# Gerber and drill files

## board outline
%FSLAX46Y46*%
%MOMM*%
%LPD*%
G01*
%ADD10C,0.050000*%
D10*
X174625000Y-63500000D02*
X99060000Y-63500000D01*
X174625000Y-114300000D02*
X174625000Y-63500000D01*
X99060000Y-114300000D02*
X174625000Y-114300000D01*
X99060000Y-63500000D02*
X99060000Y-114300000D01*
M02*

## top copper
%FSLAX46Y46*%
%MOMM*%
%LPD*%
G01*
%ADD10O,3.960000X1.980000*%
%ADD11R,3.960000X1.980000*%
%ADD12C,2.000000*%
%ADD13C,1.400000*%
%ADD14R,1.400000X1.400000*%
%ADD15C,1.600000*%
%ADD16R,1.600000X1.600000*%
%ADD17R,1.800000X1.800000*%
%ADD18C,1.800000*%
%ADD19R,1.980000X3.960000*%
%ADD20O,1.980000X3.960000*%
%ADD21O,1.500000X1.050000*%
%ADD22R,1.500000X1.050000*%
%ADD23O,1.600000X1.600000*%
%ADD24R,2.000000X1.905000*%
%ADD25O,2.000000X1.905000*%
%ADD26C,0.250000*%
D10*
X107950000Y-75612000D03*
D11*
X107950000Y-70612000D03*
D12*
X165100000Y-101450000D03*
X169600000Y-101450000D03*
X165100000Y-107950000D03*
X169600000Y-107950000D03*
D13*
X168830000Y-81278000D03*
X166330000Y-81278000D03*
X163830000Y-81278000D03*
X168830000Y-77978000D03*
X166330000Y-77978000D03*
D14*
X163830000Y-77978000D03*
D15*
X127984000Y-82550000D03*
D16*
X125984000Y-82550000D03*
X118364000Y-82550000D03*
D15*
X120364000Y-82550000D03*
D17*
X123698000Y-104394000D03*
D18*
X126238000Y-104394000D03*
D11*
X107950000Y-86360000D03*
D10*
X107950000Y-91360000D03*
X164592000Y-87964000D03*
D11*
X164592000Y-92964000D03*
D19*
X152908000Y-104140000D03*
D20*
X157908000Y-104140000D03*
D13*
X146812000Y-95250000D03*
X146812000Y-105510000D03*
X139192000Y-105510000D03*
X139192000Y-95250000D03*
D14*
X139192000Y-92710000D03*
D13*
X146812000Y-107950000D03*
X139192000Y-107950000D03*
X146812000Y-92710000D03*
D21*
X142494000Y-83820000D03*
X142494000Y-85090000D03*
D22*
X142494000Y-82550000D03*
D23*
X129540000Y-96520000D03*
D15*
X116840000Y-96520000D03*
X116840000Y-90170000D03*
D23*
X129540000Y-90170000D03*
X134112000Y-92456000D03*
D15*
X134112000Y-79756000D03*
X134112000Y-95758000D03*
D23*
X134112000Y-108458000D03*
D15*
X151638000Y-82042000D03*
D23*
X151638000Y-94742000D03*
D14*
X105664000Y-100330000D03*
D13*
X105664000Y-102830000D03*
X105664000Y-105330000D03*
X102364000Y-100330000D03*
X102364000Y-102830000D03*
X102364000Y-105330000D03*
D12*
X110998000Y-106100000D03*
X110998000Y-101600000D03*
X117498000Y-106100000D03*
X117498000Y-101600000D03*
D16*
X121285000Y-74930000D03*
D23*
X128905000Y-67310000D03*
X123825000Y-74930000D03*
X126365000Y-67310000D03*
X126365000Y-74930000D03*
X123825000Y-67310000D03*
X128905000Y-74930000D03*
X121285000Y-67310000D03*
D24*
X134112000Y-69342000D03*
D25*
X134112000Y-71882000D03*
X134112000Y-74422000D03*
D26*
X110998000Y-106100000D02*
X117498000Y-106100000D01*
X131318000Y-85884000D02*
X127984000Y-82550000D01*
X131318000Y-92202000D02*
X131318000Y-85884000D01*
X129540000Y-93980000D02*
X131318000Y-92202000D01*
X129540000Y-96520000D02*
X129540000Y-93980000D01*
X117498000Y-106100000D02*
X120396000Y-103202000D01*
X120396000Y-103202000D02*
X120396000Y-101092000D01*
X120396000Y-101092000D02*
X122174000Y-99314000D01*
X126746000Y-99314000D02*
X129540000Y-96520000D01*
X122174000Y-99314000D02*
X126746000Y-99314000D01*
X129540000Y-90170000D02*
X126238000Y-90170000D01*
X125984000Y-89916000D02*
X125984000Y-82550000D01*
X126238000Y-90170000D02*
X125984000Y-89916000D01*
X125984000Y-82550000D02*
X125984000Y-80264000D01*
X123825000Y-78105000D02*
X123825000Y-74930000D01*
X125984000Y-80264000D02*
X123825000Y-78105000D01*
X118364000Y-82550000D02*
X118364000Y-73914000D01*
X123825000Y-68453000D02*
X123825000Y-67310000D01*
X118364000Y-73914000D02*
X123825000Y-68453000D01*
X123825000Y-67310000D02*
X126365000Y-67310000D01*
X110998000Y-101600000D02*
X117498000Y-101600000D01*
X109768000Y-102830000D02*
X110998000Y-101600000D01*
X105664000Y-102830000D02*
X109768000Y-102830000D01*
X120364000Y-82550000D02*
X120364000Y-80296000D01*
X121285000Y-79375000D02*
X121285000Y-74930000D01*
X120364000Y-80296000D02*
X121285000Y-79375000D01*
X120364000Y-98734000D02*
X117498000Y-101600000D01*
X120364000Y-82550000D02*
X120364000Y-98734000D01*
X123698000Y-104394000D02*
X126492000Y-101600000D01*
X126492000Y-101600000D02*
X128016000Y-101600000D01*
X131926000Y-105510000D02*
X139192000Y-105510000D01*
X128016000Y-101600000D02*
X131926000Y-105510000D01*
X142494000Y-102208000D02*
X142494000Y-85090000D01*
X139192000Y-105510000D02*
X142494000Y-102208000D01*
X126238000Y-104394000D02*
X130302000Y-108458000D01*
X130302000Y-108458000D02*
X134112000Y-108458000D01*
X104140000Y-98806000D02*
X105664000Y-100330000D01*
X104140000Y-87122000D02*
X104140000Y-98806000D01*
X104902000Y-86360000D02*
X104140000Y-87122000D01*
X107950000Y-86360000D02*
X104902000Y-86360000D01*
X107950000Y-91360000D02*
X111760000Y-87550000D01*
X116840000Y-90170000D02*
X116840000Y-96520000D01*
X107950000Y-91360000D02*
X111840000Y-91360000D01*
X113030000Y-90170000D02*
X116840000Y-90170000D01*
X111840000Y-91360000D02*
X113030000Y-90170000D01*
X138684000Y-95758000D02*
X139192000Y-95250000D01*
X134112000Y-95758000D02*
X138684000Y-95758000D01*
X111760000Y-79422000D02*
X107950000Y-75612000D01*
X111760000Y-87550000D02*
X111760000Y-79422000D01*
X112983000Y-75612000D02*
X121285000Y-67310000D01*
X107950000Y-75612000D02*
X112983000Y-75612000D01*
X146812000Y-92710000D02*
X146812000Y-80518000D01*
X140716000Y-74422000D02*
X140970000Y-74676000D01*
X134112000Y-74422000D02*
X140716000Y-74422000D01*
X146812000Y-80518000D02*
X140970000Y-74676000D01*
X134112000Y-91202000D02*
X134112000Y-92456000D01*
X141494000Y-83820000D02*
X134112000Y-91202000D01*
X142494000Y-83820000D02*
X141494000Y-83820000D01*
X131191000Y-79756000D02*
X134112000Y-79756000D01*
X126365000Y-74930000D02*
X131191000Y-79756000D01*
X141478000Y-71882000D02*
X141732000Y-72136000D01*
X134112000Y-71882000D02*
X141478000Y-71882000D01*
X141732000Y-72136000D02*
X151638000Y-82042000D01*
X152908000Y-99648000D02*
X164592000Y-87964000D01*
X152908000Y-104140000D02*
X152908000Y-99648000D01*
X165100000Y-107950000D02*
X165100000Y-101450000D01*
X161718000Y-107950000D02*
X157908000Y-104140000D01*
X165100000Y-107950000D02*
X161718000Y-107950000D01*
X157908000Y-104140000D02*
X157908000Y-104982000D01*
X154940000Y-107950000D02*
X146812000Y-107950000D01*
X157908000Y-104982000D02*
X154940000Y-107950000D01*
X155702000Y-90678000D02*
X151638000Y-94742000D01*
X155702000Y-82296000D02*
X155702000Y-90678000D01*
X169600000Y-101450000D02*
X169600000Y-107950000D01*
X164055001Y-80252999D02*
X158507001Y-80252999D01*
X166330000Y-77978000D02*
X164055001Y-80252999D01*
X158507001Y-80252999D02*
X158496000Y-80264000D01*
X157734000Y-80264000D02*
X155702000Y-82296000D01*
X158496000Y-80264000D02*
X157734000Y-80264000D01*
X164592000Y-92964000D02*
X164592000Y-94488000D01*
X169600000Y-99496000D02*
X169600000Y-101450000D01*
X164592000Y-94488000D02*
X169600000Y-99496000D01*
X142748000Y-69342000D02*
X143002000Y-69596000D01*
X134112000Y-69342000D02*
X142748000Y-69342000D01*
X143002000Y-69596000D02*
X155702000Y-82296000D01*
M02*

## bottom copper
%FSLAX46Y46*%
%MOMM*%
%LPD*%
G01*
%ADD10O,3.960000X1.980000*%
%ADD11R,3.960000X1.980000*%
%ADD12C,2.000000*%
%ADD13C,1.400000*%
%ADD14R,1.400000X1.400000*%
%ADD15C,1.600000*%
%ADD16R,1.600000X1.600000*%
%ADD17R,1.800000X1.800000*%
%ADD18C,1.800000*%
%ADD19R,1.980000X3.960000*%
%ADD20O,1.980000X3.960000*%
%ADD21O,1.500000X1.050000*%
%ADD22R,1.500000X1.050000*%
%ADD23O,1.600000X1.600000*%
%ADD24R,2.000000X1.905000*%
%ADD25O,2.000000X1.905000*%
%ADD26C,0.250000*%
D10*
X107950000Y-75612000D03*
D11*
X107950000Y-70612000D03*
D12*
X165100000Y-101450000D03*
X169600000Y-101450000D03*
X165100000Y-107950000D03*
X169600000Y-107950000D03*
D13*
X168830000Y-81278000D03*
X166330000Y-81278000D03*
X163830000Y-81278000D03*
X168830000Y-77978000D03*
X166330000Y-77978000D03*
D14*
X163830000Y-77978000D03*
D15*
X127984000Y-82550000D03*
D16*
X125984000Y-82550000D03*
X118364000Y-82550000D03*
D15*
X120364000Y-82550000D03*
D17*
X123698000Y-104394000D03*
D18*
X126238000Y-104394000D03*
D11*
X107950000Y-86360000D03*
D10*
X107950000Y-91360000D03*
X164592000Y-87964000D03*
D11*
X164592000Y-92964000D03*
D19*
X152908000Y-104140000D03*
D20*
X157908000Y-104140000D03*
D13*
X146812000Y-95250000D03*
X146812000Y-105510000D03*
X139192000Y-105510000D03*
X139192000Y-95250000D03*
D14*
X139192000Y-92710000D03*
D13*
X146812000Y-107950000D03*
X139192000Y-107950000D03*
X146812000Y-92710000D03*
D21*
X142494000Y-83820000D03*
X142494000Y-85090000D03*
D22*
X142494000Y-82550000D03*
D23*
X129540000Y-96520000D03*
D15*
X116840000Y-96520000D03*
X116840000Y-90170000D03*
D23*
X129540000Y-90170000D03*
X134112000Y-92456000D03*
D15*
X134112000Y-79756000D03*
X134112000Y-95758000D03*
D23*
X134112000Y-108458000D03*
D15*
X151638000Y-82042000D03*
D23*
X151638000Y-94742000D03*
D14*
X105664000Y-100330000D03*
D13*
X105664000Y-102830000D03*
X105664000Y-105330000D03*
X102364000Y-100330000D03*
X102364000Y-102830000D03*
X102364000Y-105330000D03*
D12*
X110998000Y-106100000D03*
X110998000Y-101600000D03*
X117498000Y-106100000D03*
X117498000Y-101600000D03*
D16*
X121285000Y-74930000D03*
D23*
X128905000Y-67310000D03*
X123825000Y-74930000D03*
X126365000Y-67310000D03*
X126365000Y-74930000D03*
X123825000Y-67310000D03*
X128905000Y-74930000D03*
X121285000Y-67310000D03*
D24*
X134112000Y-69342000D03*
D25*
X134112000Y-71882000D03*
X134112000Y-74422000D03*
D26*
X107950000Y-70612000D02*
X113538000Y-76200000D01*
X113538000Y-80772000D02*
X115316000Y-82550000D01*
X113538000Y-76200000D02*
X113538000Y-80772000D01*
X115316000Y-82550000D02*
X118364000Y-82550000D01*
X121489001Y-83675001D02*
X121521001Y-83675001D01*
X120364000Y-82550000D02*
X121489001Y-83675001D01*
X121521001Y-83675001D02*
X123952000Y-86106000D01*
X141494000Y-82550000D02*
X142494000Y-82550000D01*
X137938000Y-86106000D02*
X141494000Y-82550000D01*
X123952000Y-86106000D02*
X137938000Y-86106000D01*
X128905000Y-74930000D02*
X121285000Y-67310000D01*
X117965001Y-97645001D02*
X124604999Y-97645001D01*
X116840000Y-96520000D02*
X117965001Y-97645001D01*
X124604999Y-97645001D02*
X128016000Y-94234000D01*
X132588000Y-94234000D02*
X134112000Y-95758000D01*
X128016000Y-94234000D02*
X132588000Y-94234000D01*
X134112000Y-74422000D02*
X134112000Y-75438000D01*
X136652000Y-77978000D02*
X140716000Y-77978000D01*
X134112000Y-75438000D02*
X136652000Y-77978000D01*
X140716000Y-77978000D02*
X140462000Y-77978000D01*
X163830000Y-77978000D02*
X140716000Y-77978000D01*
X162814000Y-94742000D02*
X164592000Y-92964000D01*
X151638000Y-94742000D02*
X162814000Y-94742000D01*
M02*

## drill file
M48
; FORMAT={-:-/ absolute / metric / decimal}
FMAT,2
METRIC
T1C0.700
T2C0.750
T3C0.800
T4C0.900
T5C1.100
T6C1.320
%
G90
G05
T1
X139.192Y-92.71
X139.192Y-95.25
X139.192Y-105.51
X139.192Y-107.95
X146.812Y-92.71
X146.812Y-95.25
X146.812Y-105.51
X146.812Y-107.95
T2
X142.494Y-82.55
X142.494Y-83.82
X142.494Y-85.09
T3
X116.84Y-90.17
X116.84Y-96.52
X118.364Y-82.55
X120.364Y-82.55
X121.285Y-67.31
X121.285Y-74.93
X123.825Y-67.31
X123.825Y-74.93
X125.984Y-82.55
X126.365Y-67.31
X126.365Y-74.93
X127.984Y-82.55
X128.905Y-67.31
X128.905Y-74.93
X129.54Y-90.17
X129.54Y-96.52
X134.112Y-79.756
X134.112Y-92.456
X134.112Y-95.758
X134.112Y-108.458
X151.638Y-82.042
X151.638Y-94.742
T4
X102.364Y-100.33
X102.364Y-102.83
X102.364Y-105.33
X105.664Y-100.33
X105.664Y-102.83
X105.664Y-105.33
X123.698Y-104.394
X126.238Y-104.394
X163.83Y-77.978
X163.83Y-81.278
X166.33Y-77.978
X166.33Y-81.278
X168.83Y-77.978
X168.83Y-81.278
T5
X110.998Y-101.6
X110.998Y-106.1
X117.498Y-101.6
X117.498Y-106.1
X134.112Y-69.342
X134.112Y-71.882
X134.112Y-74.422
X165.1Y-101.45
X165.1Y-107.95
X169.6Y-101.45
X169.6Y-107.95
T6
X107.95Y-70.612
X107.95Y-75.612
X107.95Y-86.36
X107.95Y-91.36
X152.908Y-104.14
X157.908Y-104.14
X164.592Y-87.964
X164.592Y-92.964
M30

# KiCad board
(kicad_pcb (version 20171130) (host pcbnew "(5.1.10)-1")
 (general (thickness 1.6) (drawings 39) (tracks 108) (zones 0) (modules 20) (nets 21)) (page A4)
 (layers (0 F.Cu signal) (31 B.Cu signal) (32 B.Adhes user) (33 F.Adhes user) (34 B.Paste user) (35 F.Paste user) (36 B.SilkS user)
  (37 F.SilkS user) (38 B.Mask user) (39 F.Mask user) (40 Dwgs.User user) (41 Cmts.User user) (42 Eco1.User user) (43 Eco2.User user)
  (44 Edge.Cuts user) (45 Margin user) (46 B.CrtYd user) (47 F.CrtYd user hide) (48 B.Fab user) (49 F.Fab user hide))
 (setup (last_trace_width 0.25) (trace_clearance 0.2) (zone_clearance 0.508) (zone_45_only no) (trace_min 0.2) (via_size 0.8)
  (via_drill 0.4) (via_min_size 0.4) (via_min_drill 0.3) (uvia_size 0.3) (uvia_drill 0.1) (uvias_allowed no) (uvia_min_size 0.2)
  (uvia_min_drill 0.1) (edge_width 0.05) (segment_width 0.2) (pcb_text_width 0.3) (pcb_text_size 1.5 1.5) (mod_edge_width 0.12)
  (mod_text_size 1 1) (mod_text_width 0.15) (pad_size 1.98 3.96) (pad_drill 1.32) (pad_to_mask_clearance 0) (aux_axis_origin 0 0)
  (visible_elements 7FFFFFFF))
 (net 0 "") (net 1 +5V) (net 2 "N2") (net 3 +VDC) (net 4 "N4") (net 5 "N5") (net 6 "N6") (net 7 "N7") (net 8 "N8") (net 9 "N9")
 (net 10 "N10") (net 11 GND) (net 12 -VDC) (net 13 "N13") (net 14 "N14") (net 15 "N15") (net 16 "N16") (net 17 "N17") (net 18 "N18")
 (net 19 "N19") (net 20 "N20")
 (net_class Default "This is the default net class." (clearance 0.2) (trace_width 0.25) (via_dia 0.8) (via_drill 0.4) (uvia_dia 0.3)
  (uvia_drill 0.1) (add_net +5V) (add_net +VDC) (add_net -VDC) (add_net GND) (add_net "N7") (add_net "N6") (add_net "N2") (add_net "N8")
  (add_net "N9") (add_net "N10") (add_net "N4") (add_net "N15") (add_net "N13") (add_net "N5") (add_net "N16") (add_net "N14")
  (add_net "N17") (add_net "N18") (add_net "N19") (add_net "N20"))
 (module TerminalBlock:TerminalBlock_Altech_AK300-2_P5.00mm (layer F.Cu) (at 107.95 70.612 270)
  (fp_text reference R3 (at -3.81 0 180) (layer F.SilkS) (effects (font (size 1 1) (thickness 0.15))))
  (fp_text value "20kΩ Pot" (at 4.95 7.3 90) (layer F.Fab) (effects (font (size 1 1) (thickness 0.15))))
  (pad 2 thru_hole oval (at 5 0 270) (size 1.98 3.96) (drill 1.32) (layers *.Cu *.Mask) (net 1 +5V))
  (pad 1 thru_hole rect (at 0 0 270) (size 1.98 3.96) (drill 1.32) (layers *.Cu *.Mask) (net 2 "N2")))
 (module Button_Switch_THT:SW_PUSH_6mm (layer F.Cu) (at 165.1 107.95 90)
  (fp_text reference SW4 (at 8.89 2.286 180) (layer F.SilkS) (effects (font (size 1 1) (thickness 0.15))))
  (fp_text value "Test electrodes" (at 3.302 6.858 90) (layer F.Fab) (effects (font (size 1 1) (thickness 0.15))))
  (pad 1 thru_hole circle (at 6.5 0 180) (size 2 2) (drill 1.1) (layers *.Cu *.Mask) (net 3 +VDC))
  (pad 2 thru_hole circle (at 6.5 4.5 180) (size 2 2) (drill 1.1) (layers *.Cu *.Mask) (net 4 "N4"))
  (pad 1 thru_hole circle (at 0 0 180) (size 2 2) (drill 1.1) (layers *.Cu *.Mask) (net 3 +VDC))
  (pad 2 thru_hole circle (at 0 4.5 180) (size 2 2) (drill 1.1) (layers *.Cu *.Mask) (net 4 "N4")))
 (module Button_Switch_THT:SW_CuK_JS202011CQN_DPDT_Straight (layer F.Cu) (at 163.83 77.978)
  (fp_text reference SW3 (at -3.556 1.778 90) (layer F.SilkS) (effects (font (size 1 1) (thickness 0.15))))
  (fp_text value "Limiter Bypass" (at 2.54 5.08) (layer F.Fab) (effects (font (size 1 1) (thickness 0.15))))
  (pad 6 thru_hole circle (at 5 3.3) (size 1.4 1.4) (drill 0.9) (layers *.Cu *.Mask))
  (pad 5 thru_hole circle (at 2.5 3.3) (size 1.4 1.4) (drill 0.9) (layers *.Cu *.Mask))
  (pad 4 thru_hole circle (at 0 3.3) (size 1.4 1.4) (drill 0.9) (layers *.Cu *.Mask))
  (pad 3 thru_hole circle (at 5 0) (size 1.4 1.4) (drill 0.9) (layers *.Cu *.Mask))
  (pad 2 thru_hole circle (at 2.5 0) (size 1.4 1.4) (drill 0.9) (layers *.Cu *.Mask) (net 4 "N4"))
  (pad 1 thru_hole rect (at 0 0) (size 1.4 1.4) (drill 0.9) (layers *.Cu *.Mask) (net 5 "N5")))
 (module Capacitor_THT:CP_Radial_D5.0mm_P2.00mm (layer F.Cu) (at 125.984 82.55)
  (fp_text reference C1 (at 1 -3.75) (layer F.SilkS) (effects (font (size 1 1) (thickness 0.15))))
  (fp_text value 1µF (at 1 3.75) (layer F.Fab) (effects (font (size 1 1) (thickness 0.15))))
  (pad 2 thru_hole circle (at 2 0) (size 1.6 1.6) (drill 0.8) (layers *.Cu *.Mask) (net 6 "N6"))
  (pad 1 thru_hole rect (at 0 0) (size 1.6 1.6) (drill 0.8) (layers *.Cu *.Mask) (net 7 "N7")))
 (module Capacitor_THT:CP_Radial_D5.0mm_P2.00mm (layer F.Cu) (at 118.364 82.55)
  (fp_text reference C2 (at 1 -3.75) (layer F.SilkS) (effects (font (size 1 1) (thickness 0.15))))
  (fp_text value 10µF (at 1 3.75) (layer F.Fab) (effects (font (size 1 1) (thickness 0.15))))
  (pad 1 thru_hole rect (at 0 0) (size 1.6 1.6) (drill 0.8) (layers *.Cu *.Mask) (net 2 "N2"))
  (pad 2 thru_hole circle (at 2 0) (size 1.6 1.6) (drill 0.8) (layers *.Cu *.Mask) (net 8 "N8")))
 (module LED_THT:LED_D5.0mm (layer F.Cu) (at 123.698 104.394)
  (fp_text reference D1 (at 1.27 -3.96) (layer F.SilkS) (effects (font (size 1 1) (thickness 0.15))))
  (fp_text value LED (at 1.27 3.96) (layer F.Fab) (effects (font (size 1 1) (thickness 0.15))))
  (pad 1 thru_hole rect (at 0 0) (size 1.8 1.8) (drill 0.9) (layers *.Cu *.Mask) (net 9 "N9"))
  (pad 2 thru_hole circle (at 2.54 0) (size 1.8 1.8) (drill 0.9) (layers *.Cu *.Mask) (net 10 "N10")))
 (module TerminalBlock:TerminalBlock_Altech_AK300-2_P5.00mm (layer F.Cu) (at 107.95 86.36 270)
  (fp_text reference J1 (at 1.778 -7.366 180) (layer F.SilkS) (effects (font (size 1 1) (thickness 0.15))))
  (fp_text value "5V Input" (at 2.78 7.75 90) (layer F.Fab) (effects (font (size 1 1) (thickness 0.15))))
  (pad 1 thru_hole rect (at 0 0 270) (size 1.98 3.96) (drill 1.32) (layers *.Cu *.Mask) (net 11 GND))
  (pad 2 thru_hole oval (at 5 0 270) (size 1.98 3.96) (drill 1.32) (layers *.Cu *.Mask) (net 1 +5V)))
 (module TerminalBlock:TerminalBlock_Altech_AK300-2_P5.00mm (layer F.Cu) (at 164.592 92.964 90)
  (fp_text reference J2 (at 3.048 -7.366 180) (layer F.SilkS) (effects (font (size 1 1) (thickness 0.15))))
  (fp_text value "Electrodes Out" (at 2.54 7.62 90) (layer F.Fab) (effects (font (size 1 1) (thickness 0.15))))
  (pad 2 thru_hole oval (at 5 0 90) (size 1.98 3.96) (drill 1.32) (layers *.Cu *.Mask) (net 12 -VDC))
  (pad 1 thru_hole rect (at 0 0 90) (size 1.98 3.96) (drill 1.32) (layers *.Cu *.Mask) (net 4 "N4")))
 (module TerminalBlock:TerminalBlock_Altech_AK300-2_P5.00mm (layer F.Cu) (at 152.908 104.14)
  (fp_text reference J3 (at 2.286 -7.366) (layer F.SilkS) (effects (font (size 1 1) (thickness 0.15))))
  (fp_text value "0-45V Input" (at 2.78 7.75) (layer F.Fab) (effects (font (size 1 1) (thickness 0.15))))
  (pad 1 thru_hole rect (at 0 0) (size 1.98 3.96) (drill 1.32) (layers *.Cu *.Mask) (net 12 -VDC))
  (pad 2 thru_hole oval (at 5 0) (size 1.98 3.96) (drill 1.32) (layers *.Cu *.Mask) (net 3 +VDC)))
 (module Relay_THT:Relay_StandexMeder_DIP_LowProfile (layer F.Cu) (at 139.192 92.71)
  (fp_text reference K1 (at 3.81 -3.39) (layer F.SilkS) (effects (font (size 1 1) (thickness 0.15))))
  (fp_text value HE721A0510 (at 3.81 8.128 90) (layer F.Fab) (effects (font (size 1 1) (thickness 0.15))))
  (pad 13 thru_hole circle (at 7.62 2.54) (size 1.4 1.4) (drill 0.7) (layers *.Cu *.Mask) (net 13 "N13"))
  (pad 9 thru_hole circle (at 7.62 12.8) (size 1.4 1.4) (drill 0.7) (layers *.Cu *.Mask) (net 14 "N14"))
  (pad 6 thru_hole circle (at 0 12.8) (size 1.4 1.4) (drill 0.7) (layers *.Cu *.Mask) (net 9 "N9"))
  (pad 2 thru_hole circle (at 0 2.54) (size 1.4 1.4) (drill 0.7) (layers *.Cu *.Mask) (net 1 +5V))
  (pad 1 thru_hole rect (at 0 0) (size 1.4 1.4) (drill 0.7) (layers *.Cu *.Mask) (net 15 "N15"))
  (pad 8 thru_hole circle (at 7.62 15.24) (size 1.4 1.4) (drill 0.7) (layers *.Cu *.Mask) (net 3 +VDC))
  (pad 7 thru_hole circle (at 0 15.24) (size 1.4 1.4) (drill 0.7) (layers *.Cu *.Mask) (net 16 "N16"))
  (pad 14 thru_hole circle (at 7.62 0) (size 1.4 1.4) (drill 0.7) (layers *.Cu *.Mask) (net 5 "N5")))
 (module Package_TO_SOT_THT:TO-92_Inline (layer F.Cu) (at 142.494 82.55 270)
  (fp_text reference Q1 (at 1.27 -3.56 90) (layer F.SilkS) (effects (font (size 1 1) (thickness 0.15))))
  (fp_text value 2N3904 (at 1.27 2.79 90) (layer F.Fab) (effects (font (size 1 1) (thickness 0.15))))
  (pad 2 thru_hole oval (at 1.27 0 270) (size 1.05 1.5) (drill 0.75) (layers *.Cu *.Mask) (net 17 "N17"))
  (pad 3 thru_hole oval (at 2.54 0 270) (size 1.05 1.5) (drill 0.75) (layers *.Cu *.Mask) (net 9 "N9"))
  (pad 1 thru_hole rect (at 0 0 270) (size 1.05 1.5) (drill 0.75) (layers *.Cu *.Mask) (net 8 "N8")))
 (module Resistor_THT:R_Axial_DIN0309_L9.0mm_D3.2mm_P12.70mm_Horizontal (layer F.Cu) (at 116.84 96.52)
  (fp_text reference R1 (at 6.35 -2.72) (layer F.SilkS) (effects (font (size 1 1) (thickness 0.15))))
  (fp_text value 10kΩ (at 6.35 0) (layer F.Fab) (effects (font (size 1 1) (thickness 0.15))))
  (pad 2 thru_hole oval (at 12.7 0) (size 1.6 1.6) (drill 0.8) (layers *.Cu *.Mask) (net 6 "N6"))
  (pad 1 thru_hole circle (at 0 0) (size 1.6 1.6) (drill 0.8) (layers *.Cu *.Mask) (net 1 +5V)))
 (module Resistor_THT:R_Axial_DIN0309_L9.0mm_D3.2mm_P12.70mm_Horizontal (layer F.Cu) (at 116.84 90.17)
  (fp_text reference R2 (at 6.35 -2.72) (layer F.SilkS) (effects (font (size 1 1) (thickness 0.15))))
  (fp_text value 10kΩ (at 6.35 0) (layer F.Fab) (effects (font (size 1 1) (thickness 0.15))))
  (pad 1 thru_hole circle (at 0 0) (size 1.6 1.6) (drill 0.8) (layers *.Cu *.Mask) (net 1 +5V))
  (pad 2 thru_hole oval (at 12.7 0) (size 1.6 1.6) (drill 0.8) (layers *.Cu *.Mask) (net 7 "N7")))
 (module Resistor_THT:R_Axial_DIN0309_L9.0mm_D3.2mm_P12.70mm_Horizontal (layer F.Cu) (at 134.112 79.756 270)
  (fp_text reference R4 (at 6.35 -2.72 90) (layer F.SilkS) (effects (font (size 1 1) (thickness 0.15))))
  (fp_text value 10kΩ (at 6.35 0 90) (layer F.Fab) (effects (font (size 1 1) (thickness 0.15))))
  (pad 2 thru_hole oval (at 12.7 0 270) (size 1.6 1.6) (drill 0.8) (layers *.Cu *.Mask) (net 17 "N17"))
  (pad 1 thru_hole circle (at 0 0 270) (size 1.6 1.6) (drill 0.8) (layers *.Cu *.Mask) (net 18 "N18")))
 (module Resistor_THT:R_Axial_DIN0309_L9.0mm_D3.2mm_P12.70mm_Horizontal (layer F.Cu) (at 134.112 95.758 270)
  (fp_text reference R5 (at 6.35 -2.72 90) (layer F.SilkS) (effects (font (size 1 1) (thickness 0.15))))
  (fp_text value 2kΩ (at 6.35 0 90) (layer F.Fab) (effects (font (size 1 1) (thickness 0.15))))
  (pad 1 thru_hole circle (at 0 0 270) (size 1.6 1.6) (drill 0.8) (layers *.Cu *.Mask) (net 1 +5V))
  (pad 2 thru_hole oval (at 12.7 0 270) (size 1.6 1.6) (drill 0.8) (layers *.Cu *.Mask) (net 10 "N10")))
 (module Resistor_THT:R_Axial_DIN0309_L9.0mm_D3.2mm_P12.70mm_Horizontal (layer F.Cu) (at 151.638 82.042 270)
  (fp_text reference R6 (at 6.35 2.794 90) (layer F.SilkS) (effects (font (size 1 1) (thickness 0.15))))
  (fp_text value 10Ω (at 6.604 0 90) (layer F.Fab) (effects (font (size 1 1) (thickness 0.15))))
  (pad 1 thru_hole circle (at 0 0 270) (size 1.6 1.6) (drill 0.8) (layers *.Cu *.Mask) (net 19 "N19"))
  (pad 2 thru_hole oval (at 12.7 0 270) (size 1.6 1.6) (drill 0.8) (layers *.Cu *.Mask) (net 4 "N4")))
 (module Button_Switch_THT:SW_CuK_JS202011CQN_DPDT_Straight (layer F.Cu) (at 105.664 100.33 270)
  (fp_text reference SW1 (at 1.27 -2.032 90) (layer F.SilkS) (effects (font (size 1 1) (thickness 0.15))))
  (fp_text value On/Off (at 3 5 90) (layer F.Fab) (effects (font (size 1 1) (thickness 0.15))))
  (pad 1 thru_hole rect (at 0 0 270) (size 1.4 1.4) (drill 0.9) (layers *.Cu *.Mask) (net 11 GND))
  (pad 2 thru_hole circle (at 2.5 0 270) (size 1.4 1.4) (drill 0.9) (layers *.Cu *.Mask) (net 8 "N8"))
  (pad 3 thru_hole circle (at 5 0 270) (size 1.4 1.4) (drill 0.9) (layers *.Cu *.Mask))
  (pad 4 thru_hole circle (at 0 3.3 270) (size 1.4 1.4) (drill 0.9) (layers *.Cu *.Mask))
  (pad 5 thru_hole circle (at 2.5 3.3 270) (size 1.4 1.4) (drill 0.9) (layers *.Cu *.Mask))
  (pad 6 thru_hole circle (at 5 3.3 270) (size 1.4 1.4) (drill 0.9) (layers *.Cu *.Mask)))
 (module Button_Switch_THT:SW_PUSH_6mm (layer F.Cu) (at 110.998 101.6)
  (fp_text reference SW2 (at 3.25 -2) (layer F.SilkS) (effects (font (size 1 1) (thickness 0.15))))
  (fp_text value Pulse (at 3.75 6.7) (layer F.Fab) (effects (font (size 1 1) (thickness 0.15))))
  (pad 2 thru_hole circle (at 0 4.5 90) (size 2 2) (drill 1.1) (layers *.Cu *.Mask) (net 6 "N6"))
  (pad 1 thru_hole circle (at 0 0 90) (size 2 2) (drill 1.1) (layers *.Cu *.Mask) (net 8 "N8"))
  (pad 2 thru_hole circle (at 6.5 4.5 90) (size 2 2) (drill 1.1) (layers *.Cu *.Mask) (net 6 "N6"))
  (pad 1 thru_hole circle (at 6.5 0 90) (size 2 2) (drill 1.1) (layers *.Cu *.Mask) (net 8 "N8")))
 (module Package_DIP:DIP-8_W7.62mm (layer F.Cu) (at 121.285 74.93 90)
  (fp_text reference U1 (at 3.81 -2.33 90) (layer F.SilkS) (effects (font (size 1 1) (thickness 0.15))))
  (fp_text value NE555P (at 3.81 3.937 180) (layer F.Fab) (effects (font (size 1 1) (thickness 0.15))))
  (pad 1 thru_hole rect (at 0 0 90) (size 1.6 1.6) (drill 0.8) (layers *.Cu *.Mask) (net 8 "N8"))
  (pad 5 thru_hole oval (at 7.62 7.62 90) (size 1.6 1.6) (drill 0.8) (layers *.Cu *.Mask) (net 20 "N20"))
  (pad 2 thru_hole oval (at 0 2.54 90) (size 1.6 1.6) (drill 0.8) (layers *.Cu *.Mask) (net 7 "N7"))
  (pad 6 thru_hole oval (at 7.62 5.08 90) (size 1.6 1.6) (drill 0.8) (layers *.Cu *.Mask) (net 2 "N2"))
  (pad 3 thru_hole oval (at 0 5.08 90) (size 1.6 1.6) (drill 0.8) (layers *.Cu *.Mask) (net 18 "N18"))
  (pad 7 thru_hole oval (at 7.62 2.54 90) (size 1.6 1.6) (drill 0.8) (layers *.Cu *.Mask) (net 2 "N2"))
  (pad 4 thru_hole oval (at 0 7.62 90) (size 1.6 1.6) (drill 0.8) (layers *.Cu *.Mask) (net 1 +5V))
  (pad 8 thru_hole oval (at 7.62 0 90) (size 1.6 1.6) (drill 0.8) (layers *.Cu *.Mask) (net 1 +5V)))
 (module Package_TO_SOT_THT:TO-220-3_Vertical (layer F.Cu) (at 134.112 69.342 270)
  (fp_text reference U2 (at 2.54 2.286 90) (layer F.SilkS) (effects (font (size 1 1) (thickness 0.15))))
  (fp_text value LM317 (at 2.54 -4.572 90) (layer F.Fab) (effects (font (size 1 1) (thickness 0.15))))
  (pad 1 thru_hole rect (at 0 0 270) (size 1.905 2) (drill 1.1) (layers *.Cu *.Mask) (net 4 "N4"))
  (pad 2 thru_hole oval (at 2.54 0 270) (size 1.905 2) (drill 1.1) (layers *.Cu *.Mask) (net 19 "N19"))
  (pad 3 thru_hole oval (at 5.08 0 270) (size 1.905 2) (drill 1.1) (layers *.Cu *.Mask) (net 5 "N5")))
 (gr_line (start 174.625 63.5) (end 99.06 63.5) (layer Edge.Cuts) (width 0.05))
 (gr_line (start 174.625 114.3) (end 174.625 63.5) (layer Edge.Cuts) (width 0.05))
 (gr_line (start 99.06 114.3) (end 174.625 114.3) (layer Edge.Cuts) (width 0.05))
 (gr_line (start 99.06 63.5) (end 99.06 114.3) (layer Edge.Cuts) (width 0.05))
 (segment (start 110.998 106.1) (end 117.498 106.1) (width 0.25) (layer F.Cu) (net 6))
 (segment (start 131.318 85.884) (end 127.984 82.55) (width 0.25) (layer F.Cu) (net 6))
 (segment (start 131.318 92.202) (end 131.318 85.884) (width 0.25) (layer F.Cu) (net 6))
 (segment (start 129.54 93.98) (end 131.318 92.202) (width 0.25) (layer F.Cu) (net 6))
 (segment (start 129.54 96.52) (end 129.54 93.98) (width 0.25) (layer F.Cu) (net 6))
 (segment (start 117.498 106.1) (end 120.396 103.202) (width 0.25) (layer F.Cu) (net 6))
 (segment (start 120.396 103.202) (end 120.396 101.092) (width 0.25) (layer F.Cu) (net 6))
 (segment (start 120.396 101.092) (end 122.174 99.314) (width 0.25) (layer F.Cu) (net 6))
 (segment (start 126.746 99.314) (end 129.54 96.52) (width 0.25) (layer F.Cu) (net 6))
 (segment (start 122.174 99.314) (end 126.746 99.314) (width 0.25) (layer F.Cu) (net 6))
 (segment (start 129.54 90.17) (end 126.238 90.17) (width 0.25) (layer F.Cu) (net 7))
 (segment (start 125.984 89.916) (end 125.984 82.55) (width 0.25) (layer F.Cu) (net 7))
 (segment (start 126.238 90.17) (end 125.984 89.916) (width 0.25) (layer F.Cu) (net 7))
 (segment (start 125.984 82.55) (end 125.984 80.264) (width 0.25) (layer F.Cu) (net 7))
 (segment (start 123.825 78.105) (end 123.825 74.93) (width 0.25) (layer F.Cu) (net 7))
 (segment (start 125.984 80.264) (end 123.825 78.105) (width 0.25) (layer F.Cu) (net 7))
 (segment (start 118.364 82.55) (end 118.364 73.914) (width 0.25) (layer F.Cu) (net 2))
 (segment (start 123.825 68.453) (end 123.825 67.31) (width 0.25) (layer F.Cu) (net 2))
 (segment (start 118.364 73.914) (end 123.825 68.453) (width 0.25) (layer F.Cu) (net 2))
 (segment (start 123.825 67.31) (end 126.365 67.31) (width 0.25) (layer F.Cu) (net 2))
 (segment (start 107.95 70.612) (end 113.538 76.2) (width 0.25) (layer B.Cu) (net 2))
 (segment (start 113.538 80.772) (end 115.316 82.55) (width 0.25) (layer B.Cu) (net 2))
 (segment (start 113.538 76.2) (end 113.538 80.772) (width 0.25) (layer B.Cu) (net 2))
 (segment (start 115.316 82.55) (end 118.364 82.55) (width 0.25) (layer B.Cu) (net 2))
 (segment (start 110.998 101.6) (end 117.498 101.6) (width 0.25) (layer F.Cu) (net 8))
 (segment (start 109.768 102.83) (end 110.998 101.6) (width 0.25) (layer F.Cu) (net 8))
 (segment (start 105.664 102.83) (end 109.768 102.83) (width 0.25) (layer F.Cu) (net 8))
 (segment (start 120.364 82.55) (end 120.364 80.296) (width 0.25) (layer F.Cu) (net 8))
 (segment (start 121.285 79.375) (end 121.285 74.93) (width 0.25) (layer F.Cu) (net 8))
 (segment (start 120.364 80.296) (end 121.285 79.375) (width 0.25) (layer F.Cu) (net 8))
 (segment (start 120.364 98.734) (end 117.498 101.6) (width 0.25) (layer F.Cu) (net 8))
 (segment (start 120.364 82.55) (end 120.364 98.734) (width 0.25) (layer F.Cu) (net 8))
 (segment (start 121.489001 83.675001) (end 121.521001 83.675001) (width 0.25) (layer B.Cu) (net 8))
 (segment (start 120.364 82.55) (end 121.489001 83.675001) (width 0.25) (layer B.Cu) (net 8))
 (segment (start 121.521001 83.675001) (end 123.952 86.106) (width 0.25) (layer B.Cu) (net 8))
 (segment (start 141.494 82.55) (end 142.494 82.55) (width 0.25) (layer B.Cu) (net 8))
 (segment (start 137.938 86.106) (end 141.494 82.55) (width 0.25) (layer B.Cu) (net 8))
 (segment (start 123.952 86.106) (end 137.938 86.106) (width 0.25) (layer B.Cu) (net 8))
 (segment (start 123.698 104.394) (end 126.492 101.6) (width 0.25) (layer F.Cu) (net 9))
 (segment (start 126.492 101.6) (end 128.016 101.6) (width 0.25) (layer F.Cu) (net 9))
 (segment (start 131.926 105.51) (end 139.192 105.51) (width 0.25) (layer F.Cu) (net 9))
 (segment (start 128.016 101.6) (end 131.926 105.51) (width 0.25) (layer F.Cu) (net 9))
 (segment (start 142.494 102.208) (end 142.494 85.09) (width 0.25) (layer F.Cu) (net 9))
 (segment (start 139.192 105.51) (end 142.494 102.208) (width 0.25) (layer F.Cu) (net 9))
 (segment (start 126.238 104.394) (end 130.302 108.458) (width 0.25) (layer F.Cu) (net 10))
 (segment (start 130.302 108.458) (end 134.112 108.458) (width 0.25) (layer F.Cu) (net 10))
 (segment (start 104.14 98.806) (end 105.664 100.33) (width 0.25) (layer F.Cu) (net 11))
 (segment (start 104.14 87.122) (end 104.14 98.806) (width 0.25) (layer F.Cu) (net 11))
 (segment (start 104.902 86.36) (end 104.14 87.122) (width 0.25) (layer F.Cu) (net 11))
 (segment (start 107.95 86.36) (end 104.902 86.36) (width 0.25) (layer F.Cu) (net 11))
 (segment (start 107.95 91.36) (end 111.76 87.55) (width 0.25) (layer F.Cu) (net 1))
 (segment (start 116.84 90.17) (end 116.84 96.52) (width 0.25) (layer F.Cu) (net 1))
 (segment (start 107.95 91.36) (end 111.84 91.36) (width 0.25) (layer F.Cu) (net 1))
 (segment (start 113.03 90.17) (end 116.84 90.17) (width 0.25) (layer F.Cu) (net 1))
 (segment (start 111.84 91.36) (end 113.03 90.17) (width 0.25) (layer F.Cu) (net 1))
 (segment (start 138.684 95.758) (end 139.192 95.25) (width 0.25) (layer F.Cu) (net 1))
 (segment (start 134.112 95.758) (end 138.684 95.758) (width 0.25) (layer F.Cu) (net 1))
 (segment (start 128.905 74.93) (end 121.285 67.31) (width 0.25) (layer B.Cu) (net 1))
 (segment (start 117.965001 97.645001) (end 124.604999 97.645001) (width 0.25) (layer B.Cu) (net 1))
 (segment (start 116.84 96.52) (end 117.965001 97.645001) (width 0.25) (layer B.Cu) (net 1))
 (segment (start 124.604999 97.645001) (end 128.016 94.234) (width 0.25) (layer B.Cu) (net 1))
 (segment (start 132.588 94.234) (end 134.112 95.758) (width 0.25) (layer B.Cu) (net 1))
 (segment (start 128.016 94.234) (end 132.588 94.234) (width 0.25) (layer B.Cu) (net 1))
 (segment (start 111.76 79.422) (end 107.95 75.612) (width 0.25) (layer F.Cu) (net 1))
 (segment (start 111.76 87.55) (end 111.76 79.422) (width 0.25) (layer F.Cu) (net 1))
 (segment (start 112.983 75.612) (end 121.285 67.31) (width 0.25) (layer F.Cu) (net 1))
 (segment (start 107.95 75.612) (end 112.983 75.612) (width 0.25) (layer F.Cu) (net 1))
 (segment (start 146.812 92.71) (end 146.812 80.518) (width 0.25) (layer F.Cu) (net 5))
 (segment (start 140.716 74.422) (end 140.97 74.676) (width 0.25) (layer F.Cu) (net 5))
 (segment (start 134.112 74.422) (end 140.716 74.422) (width 0.25) (layer F.Cu) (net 5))
 (segment (start 146.812 80.518) (end 140.97 74.676) (width 0.25) (layer F.Cu) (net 5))
 (segment (start 134.112 74.422) (end 134.112 75.438) (width 0.25) (layer B.Cu) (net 5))
 (segment (start 136.652 77.978) (end 140.716 77.978) (width 0.25) (layer B.Cu) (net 5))
 (segment (start 134.112 75.438) (end 136.652 77.978) (width 0.25) (layer B.Cu) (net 5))
 (segment (start 140.716 77.978) (end 140.462 77.978) (width 0.25) (layer B.Cu) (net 5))
 (segment (start 163.83 77.978) (end 140.716 77.978) (width 0.25) (layer B.Cu) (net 5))
 (segment (start 134.112 91.202) (end 134.112 92.456) (width 0.25) (layer F.Cu) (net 17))
 (segment (start 141.494 83.82) (end 134.112 91.202) (width 0.25) (layer F.Cu) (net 17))
 (segment (start 142.494 83.82) (end 141.494 83.82) (width 0.25) (layer F.Cu) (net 17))
 (segment (start 131.191 79.756) (end 134.112 79.756) (width 0.25) (layer F.Cu) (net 18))
 (segment (start 126.365 74.93) (end 131.191 79.756) (width 0.25) (layer F.Cu) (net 18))
 (segment (start 141.478 71.882) (end 141.732 72.136) (width 0.25) (layer F.Cu) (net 19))
 (segment (start 134.112 71.882) (end 141.478 71.882) (width 0.25) (layer F.Cu) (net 19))
 (segment (start 141.732 72.136) (end 151.638 82.042) (width 0.25) (layer F.Cu) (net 19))
 (segment (start 152.908 99.648) (end 164.592 87.964) (width 0.25) (layer F.Cu) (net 12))
 (segment (start 152.908 104.14) (end 152.908 99.648) (width 0.25) (layer F.Cu) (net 12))
 (segment (start 165.1 107.95) (end 165.1 101.45) (width 0.25) (layer F.Cu) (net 3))
 (segment (start 161.718 107.95) (end 157.908 104.14) (width 0.25) (layer F.Cu) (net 3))
 (segment (start 165.1 107.95) (end 161.718 107.95) (width 0.25) (layer F.Cu) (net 3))
 (segment (start 157.908 104.14) (end 157.908 104.982) (width 0.25) (layer F.Cu) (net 3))
 (segment (start 154.94 107.95) (end 146.812 107.95) (width 0.25) (layer F.Cu) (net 3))
 (segment (start 157.908 104.982) (end 154.94 107.95) (width 0.25) (layer F.Cu) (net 3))
 (segment (start 155.702 90.678) (end 151.638 94.742) (width 0.25) (layer F.Cu) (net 4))
 (segment (start 155.702 82.296) (end 155.702 90.678) (width 0.25) (layer F.Cu) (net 4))
 (segment (start 169.6 101.45) (end 169.6 107.95) (width 0.25) (layer F.Cu) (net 4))
 (segment (start 164.055001 80.252999) (end 158.507001 80.252999) (width 0.25) (layer F.Cu) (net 4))
 (segment (start 166.33 77.978) (end 164.055001 80.252999) (width 0.25) (layer F.Cu) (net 4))
 (segment (start 158.507001 80.252999) (end 158.496 80.264) (width 0.25) (layer F.Cu) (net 4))
 (segment (start 157.734 80.264) (end 155.702 82.296) (width 0.25) (layer F.Cu) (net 4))
 (segment (start 158.496 80.264) (end 157.734 80.264) (width 0.25) (layer F.Cu) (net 4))
 (segment (start 164.592 92.964) (end 164.592 94.488) (width 0.25) (layer F.Cu) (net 4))
 (segment (start 169.6 99.496) (end 169.6 101.45) (width 0.25) (layer F.Cu) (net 4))
 (segment (start 164.592 94.488) (end 169.6 99.496) (width 0.25) (layer F.Cu) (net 4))
 (segment (start 162.814 94.742) (end 164.592 92.964) (width 0.25) (layer B.Cu) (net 4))
 (segment (start 151.638 94.742) (end 162.814 94.742) (width 0.25) (layer B.Cu) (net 4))
 (segment (start 142.748 69.342) (end 143.002 69.596) (width 0.25) (layer F.Cu) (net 4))
 (segment (start 134.112 69.342) (end 142.748 69.342) (width 0.25) (layer F.Cu) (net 4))
 (segment (start 143.002 69.596) (end 155.702 82.296) (width 0.25) (layer F.Cu) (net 4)))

